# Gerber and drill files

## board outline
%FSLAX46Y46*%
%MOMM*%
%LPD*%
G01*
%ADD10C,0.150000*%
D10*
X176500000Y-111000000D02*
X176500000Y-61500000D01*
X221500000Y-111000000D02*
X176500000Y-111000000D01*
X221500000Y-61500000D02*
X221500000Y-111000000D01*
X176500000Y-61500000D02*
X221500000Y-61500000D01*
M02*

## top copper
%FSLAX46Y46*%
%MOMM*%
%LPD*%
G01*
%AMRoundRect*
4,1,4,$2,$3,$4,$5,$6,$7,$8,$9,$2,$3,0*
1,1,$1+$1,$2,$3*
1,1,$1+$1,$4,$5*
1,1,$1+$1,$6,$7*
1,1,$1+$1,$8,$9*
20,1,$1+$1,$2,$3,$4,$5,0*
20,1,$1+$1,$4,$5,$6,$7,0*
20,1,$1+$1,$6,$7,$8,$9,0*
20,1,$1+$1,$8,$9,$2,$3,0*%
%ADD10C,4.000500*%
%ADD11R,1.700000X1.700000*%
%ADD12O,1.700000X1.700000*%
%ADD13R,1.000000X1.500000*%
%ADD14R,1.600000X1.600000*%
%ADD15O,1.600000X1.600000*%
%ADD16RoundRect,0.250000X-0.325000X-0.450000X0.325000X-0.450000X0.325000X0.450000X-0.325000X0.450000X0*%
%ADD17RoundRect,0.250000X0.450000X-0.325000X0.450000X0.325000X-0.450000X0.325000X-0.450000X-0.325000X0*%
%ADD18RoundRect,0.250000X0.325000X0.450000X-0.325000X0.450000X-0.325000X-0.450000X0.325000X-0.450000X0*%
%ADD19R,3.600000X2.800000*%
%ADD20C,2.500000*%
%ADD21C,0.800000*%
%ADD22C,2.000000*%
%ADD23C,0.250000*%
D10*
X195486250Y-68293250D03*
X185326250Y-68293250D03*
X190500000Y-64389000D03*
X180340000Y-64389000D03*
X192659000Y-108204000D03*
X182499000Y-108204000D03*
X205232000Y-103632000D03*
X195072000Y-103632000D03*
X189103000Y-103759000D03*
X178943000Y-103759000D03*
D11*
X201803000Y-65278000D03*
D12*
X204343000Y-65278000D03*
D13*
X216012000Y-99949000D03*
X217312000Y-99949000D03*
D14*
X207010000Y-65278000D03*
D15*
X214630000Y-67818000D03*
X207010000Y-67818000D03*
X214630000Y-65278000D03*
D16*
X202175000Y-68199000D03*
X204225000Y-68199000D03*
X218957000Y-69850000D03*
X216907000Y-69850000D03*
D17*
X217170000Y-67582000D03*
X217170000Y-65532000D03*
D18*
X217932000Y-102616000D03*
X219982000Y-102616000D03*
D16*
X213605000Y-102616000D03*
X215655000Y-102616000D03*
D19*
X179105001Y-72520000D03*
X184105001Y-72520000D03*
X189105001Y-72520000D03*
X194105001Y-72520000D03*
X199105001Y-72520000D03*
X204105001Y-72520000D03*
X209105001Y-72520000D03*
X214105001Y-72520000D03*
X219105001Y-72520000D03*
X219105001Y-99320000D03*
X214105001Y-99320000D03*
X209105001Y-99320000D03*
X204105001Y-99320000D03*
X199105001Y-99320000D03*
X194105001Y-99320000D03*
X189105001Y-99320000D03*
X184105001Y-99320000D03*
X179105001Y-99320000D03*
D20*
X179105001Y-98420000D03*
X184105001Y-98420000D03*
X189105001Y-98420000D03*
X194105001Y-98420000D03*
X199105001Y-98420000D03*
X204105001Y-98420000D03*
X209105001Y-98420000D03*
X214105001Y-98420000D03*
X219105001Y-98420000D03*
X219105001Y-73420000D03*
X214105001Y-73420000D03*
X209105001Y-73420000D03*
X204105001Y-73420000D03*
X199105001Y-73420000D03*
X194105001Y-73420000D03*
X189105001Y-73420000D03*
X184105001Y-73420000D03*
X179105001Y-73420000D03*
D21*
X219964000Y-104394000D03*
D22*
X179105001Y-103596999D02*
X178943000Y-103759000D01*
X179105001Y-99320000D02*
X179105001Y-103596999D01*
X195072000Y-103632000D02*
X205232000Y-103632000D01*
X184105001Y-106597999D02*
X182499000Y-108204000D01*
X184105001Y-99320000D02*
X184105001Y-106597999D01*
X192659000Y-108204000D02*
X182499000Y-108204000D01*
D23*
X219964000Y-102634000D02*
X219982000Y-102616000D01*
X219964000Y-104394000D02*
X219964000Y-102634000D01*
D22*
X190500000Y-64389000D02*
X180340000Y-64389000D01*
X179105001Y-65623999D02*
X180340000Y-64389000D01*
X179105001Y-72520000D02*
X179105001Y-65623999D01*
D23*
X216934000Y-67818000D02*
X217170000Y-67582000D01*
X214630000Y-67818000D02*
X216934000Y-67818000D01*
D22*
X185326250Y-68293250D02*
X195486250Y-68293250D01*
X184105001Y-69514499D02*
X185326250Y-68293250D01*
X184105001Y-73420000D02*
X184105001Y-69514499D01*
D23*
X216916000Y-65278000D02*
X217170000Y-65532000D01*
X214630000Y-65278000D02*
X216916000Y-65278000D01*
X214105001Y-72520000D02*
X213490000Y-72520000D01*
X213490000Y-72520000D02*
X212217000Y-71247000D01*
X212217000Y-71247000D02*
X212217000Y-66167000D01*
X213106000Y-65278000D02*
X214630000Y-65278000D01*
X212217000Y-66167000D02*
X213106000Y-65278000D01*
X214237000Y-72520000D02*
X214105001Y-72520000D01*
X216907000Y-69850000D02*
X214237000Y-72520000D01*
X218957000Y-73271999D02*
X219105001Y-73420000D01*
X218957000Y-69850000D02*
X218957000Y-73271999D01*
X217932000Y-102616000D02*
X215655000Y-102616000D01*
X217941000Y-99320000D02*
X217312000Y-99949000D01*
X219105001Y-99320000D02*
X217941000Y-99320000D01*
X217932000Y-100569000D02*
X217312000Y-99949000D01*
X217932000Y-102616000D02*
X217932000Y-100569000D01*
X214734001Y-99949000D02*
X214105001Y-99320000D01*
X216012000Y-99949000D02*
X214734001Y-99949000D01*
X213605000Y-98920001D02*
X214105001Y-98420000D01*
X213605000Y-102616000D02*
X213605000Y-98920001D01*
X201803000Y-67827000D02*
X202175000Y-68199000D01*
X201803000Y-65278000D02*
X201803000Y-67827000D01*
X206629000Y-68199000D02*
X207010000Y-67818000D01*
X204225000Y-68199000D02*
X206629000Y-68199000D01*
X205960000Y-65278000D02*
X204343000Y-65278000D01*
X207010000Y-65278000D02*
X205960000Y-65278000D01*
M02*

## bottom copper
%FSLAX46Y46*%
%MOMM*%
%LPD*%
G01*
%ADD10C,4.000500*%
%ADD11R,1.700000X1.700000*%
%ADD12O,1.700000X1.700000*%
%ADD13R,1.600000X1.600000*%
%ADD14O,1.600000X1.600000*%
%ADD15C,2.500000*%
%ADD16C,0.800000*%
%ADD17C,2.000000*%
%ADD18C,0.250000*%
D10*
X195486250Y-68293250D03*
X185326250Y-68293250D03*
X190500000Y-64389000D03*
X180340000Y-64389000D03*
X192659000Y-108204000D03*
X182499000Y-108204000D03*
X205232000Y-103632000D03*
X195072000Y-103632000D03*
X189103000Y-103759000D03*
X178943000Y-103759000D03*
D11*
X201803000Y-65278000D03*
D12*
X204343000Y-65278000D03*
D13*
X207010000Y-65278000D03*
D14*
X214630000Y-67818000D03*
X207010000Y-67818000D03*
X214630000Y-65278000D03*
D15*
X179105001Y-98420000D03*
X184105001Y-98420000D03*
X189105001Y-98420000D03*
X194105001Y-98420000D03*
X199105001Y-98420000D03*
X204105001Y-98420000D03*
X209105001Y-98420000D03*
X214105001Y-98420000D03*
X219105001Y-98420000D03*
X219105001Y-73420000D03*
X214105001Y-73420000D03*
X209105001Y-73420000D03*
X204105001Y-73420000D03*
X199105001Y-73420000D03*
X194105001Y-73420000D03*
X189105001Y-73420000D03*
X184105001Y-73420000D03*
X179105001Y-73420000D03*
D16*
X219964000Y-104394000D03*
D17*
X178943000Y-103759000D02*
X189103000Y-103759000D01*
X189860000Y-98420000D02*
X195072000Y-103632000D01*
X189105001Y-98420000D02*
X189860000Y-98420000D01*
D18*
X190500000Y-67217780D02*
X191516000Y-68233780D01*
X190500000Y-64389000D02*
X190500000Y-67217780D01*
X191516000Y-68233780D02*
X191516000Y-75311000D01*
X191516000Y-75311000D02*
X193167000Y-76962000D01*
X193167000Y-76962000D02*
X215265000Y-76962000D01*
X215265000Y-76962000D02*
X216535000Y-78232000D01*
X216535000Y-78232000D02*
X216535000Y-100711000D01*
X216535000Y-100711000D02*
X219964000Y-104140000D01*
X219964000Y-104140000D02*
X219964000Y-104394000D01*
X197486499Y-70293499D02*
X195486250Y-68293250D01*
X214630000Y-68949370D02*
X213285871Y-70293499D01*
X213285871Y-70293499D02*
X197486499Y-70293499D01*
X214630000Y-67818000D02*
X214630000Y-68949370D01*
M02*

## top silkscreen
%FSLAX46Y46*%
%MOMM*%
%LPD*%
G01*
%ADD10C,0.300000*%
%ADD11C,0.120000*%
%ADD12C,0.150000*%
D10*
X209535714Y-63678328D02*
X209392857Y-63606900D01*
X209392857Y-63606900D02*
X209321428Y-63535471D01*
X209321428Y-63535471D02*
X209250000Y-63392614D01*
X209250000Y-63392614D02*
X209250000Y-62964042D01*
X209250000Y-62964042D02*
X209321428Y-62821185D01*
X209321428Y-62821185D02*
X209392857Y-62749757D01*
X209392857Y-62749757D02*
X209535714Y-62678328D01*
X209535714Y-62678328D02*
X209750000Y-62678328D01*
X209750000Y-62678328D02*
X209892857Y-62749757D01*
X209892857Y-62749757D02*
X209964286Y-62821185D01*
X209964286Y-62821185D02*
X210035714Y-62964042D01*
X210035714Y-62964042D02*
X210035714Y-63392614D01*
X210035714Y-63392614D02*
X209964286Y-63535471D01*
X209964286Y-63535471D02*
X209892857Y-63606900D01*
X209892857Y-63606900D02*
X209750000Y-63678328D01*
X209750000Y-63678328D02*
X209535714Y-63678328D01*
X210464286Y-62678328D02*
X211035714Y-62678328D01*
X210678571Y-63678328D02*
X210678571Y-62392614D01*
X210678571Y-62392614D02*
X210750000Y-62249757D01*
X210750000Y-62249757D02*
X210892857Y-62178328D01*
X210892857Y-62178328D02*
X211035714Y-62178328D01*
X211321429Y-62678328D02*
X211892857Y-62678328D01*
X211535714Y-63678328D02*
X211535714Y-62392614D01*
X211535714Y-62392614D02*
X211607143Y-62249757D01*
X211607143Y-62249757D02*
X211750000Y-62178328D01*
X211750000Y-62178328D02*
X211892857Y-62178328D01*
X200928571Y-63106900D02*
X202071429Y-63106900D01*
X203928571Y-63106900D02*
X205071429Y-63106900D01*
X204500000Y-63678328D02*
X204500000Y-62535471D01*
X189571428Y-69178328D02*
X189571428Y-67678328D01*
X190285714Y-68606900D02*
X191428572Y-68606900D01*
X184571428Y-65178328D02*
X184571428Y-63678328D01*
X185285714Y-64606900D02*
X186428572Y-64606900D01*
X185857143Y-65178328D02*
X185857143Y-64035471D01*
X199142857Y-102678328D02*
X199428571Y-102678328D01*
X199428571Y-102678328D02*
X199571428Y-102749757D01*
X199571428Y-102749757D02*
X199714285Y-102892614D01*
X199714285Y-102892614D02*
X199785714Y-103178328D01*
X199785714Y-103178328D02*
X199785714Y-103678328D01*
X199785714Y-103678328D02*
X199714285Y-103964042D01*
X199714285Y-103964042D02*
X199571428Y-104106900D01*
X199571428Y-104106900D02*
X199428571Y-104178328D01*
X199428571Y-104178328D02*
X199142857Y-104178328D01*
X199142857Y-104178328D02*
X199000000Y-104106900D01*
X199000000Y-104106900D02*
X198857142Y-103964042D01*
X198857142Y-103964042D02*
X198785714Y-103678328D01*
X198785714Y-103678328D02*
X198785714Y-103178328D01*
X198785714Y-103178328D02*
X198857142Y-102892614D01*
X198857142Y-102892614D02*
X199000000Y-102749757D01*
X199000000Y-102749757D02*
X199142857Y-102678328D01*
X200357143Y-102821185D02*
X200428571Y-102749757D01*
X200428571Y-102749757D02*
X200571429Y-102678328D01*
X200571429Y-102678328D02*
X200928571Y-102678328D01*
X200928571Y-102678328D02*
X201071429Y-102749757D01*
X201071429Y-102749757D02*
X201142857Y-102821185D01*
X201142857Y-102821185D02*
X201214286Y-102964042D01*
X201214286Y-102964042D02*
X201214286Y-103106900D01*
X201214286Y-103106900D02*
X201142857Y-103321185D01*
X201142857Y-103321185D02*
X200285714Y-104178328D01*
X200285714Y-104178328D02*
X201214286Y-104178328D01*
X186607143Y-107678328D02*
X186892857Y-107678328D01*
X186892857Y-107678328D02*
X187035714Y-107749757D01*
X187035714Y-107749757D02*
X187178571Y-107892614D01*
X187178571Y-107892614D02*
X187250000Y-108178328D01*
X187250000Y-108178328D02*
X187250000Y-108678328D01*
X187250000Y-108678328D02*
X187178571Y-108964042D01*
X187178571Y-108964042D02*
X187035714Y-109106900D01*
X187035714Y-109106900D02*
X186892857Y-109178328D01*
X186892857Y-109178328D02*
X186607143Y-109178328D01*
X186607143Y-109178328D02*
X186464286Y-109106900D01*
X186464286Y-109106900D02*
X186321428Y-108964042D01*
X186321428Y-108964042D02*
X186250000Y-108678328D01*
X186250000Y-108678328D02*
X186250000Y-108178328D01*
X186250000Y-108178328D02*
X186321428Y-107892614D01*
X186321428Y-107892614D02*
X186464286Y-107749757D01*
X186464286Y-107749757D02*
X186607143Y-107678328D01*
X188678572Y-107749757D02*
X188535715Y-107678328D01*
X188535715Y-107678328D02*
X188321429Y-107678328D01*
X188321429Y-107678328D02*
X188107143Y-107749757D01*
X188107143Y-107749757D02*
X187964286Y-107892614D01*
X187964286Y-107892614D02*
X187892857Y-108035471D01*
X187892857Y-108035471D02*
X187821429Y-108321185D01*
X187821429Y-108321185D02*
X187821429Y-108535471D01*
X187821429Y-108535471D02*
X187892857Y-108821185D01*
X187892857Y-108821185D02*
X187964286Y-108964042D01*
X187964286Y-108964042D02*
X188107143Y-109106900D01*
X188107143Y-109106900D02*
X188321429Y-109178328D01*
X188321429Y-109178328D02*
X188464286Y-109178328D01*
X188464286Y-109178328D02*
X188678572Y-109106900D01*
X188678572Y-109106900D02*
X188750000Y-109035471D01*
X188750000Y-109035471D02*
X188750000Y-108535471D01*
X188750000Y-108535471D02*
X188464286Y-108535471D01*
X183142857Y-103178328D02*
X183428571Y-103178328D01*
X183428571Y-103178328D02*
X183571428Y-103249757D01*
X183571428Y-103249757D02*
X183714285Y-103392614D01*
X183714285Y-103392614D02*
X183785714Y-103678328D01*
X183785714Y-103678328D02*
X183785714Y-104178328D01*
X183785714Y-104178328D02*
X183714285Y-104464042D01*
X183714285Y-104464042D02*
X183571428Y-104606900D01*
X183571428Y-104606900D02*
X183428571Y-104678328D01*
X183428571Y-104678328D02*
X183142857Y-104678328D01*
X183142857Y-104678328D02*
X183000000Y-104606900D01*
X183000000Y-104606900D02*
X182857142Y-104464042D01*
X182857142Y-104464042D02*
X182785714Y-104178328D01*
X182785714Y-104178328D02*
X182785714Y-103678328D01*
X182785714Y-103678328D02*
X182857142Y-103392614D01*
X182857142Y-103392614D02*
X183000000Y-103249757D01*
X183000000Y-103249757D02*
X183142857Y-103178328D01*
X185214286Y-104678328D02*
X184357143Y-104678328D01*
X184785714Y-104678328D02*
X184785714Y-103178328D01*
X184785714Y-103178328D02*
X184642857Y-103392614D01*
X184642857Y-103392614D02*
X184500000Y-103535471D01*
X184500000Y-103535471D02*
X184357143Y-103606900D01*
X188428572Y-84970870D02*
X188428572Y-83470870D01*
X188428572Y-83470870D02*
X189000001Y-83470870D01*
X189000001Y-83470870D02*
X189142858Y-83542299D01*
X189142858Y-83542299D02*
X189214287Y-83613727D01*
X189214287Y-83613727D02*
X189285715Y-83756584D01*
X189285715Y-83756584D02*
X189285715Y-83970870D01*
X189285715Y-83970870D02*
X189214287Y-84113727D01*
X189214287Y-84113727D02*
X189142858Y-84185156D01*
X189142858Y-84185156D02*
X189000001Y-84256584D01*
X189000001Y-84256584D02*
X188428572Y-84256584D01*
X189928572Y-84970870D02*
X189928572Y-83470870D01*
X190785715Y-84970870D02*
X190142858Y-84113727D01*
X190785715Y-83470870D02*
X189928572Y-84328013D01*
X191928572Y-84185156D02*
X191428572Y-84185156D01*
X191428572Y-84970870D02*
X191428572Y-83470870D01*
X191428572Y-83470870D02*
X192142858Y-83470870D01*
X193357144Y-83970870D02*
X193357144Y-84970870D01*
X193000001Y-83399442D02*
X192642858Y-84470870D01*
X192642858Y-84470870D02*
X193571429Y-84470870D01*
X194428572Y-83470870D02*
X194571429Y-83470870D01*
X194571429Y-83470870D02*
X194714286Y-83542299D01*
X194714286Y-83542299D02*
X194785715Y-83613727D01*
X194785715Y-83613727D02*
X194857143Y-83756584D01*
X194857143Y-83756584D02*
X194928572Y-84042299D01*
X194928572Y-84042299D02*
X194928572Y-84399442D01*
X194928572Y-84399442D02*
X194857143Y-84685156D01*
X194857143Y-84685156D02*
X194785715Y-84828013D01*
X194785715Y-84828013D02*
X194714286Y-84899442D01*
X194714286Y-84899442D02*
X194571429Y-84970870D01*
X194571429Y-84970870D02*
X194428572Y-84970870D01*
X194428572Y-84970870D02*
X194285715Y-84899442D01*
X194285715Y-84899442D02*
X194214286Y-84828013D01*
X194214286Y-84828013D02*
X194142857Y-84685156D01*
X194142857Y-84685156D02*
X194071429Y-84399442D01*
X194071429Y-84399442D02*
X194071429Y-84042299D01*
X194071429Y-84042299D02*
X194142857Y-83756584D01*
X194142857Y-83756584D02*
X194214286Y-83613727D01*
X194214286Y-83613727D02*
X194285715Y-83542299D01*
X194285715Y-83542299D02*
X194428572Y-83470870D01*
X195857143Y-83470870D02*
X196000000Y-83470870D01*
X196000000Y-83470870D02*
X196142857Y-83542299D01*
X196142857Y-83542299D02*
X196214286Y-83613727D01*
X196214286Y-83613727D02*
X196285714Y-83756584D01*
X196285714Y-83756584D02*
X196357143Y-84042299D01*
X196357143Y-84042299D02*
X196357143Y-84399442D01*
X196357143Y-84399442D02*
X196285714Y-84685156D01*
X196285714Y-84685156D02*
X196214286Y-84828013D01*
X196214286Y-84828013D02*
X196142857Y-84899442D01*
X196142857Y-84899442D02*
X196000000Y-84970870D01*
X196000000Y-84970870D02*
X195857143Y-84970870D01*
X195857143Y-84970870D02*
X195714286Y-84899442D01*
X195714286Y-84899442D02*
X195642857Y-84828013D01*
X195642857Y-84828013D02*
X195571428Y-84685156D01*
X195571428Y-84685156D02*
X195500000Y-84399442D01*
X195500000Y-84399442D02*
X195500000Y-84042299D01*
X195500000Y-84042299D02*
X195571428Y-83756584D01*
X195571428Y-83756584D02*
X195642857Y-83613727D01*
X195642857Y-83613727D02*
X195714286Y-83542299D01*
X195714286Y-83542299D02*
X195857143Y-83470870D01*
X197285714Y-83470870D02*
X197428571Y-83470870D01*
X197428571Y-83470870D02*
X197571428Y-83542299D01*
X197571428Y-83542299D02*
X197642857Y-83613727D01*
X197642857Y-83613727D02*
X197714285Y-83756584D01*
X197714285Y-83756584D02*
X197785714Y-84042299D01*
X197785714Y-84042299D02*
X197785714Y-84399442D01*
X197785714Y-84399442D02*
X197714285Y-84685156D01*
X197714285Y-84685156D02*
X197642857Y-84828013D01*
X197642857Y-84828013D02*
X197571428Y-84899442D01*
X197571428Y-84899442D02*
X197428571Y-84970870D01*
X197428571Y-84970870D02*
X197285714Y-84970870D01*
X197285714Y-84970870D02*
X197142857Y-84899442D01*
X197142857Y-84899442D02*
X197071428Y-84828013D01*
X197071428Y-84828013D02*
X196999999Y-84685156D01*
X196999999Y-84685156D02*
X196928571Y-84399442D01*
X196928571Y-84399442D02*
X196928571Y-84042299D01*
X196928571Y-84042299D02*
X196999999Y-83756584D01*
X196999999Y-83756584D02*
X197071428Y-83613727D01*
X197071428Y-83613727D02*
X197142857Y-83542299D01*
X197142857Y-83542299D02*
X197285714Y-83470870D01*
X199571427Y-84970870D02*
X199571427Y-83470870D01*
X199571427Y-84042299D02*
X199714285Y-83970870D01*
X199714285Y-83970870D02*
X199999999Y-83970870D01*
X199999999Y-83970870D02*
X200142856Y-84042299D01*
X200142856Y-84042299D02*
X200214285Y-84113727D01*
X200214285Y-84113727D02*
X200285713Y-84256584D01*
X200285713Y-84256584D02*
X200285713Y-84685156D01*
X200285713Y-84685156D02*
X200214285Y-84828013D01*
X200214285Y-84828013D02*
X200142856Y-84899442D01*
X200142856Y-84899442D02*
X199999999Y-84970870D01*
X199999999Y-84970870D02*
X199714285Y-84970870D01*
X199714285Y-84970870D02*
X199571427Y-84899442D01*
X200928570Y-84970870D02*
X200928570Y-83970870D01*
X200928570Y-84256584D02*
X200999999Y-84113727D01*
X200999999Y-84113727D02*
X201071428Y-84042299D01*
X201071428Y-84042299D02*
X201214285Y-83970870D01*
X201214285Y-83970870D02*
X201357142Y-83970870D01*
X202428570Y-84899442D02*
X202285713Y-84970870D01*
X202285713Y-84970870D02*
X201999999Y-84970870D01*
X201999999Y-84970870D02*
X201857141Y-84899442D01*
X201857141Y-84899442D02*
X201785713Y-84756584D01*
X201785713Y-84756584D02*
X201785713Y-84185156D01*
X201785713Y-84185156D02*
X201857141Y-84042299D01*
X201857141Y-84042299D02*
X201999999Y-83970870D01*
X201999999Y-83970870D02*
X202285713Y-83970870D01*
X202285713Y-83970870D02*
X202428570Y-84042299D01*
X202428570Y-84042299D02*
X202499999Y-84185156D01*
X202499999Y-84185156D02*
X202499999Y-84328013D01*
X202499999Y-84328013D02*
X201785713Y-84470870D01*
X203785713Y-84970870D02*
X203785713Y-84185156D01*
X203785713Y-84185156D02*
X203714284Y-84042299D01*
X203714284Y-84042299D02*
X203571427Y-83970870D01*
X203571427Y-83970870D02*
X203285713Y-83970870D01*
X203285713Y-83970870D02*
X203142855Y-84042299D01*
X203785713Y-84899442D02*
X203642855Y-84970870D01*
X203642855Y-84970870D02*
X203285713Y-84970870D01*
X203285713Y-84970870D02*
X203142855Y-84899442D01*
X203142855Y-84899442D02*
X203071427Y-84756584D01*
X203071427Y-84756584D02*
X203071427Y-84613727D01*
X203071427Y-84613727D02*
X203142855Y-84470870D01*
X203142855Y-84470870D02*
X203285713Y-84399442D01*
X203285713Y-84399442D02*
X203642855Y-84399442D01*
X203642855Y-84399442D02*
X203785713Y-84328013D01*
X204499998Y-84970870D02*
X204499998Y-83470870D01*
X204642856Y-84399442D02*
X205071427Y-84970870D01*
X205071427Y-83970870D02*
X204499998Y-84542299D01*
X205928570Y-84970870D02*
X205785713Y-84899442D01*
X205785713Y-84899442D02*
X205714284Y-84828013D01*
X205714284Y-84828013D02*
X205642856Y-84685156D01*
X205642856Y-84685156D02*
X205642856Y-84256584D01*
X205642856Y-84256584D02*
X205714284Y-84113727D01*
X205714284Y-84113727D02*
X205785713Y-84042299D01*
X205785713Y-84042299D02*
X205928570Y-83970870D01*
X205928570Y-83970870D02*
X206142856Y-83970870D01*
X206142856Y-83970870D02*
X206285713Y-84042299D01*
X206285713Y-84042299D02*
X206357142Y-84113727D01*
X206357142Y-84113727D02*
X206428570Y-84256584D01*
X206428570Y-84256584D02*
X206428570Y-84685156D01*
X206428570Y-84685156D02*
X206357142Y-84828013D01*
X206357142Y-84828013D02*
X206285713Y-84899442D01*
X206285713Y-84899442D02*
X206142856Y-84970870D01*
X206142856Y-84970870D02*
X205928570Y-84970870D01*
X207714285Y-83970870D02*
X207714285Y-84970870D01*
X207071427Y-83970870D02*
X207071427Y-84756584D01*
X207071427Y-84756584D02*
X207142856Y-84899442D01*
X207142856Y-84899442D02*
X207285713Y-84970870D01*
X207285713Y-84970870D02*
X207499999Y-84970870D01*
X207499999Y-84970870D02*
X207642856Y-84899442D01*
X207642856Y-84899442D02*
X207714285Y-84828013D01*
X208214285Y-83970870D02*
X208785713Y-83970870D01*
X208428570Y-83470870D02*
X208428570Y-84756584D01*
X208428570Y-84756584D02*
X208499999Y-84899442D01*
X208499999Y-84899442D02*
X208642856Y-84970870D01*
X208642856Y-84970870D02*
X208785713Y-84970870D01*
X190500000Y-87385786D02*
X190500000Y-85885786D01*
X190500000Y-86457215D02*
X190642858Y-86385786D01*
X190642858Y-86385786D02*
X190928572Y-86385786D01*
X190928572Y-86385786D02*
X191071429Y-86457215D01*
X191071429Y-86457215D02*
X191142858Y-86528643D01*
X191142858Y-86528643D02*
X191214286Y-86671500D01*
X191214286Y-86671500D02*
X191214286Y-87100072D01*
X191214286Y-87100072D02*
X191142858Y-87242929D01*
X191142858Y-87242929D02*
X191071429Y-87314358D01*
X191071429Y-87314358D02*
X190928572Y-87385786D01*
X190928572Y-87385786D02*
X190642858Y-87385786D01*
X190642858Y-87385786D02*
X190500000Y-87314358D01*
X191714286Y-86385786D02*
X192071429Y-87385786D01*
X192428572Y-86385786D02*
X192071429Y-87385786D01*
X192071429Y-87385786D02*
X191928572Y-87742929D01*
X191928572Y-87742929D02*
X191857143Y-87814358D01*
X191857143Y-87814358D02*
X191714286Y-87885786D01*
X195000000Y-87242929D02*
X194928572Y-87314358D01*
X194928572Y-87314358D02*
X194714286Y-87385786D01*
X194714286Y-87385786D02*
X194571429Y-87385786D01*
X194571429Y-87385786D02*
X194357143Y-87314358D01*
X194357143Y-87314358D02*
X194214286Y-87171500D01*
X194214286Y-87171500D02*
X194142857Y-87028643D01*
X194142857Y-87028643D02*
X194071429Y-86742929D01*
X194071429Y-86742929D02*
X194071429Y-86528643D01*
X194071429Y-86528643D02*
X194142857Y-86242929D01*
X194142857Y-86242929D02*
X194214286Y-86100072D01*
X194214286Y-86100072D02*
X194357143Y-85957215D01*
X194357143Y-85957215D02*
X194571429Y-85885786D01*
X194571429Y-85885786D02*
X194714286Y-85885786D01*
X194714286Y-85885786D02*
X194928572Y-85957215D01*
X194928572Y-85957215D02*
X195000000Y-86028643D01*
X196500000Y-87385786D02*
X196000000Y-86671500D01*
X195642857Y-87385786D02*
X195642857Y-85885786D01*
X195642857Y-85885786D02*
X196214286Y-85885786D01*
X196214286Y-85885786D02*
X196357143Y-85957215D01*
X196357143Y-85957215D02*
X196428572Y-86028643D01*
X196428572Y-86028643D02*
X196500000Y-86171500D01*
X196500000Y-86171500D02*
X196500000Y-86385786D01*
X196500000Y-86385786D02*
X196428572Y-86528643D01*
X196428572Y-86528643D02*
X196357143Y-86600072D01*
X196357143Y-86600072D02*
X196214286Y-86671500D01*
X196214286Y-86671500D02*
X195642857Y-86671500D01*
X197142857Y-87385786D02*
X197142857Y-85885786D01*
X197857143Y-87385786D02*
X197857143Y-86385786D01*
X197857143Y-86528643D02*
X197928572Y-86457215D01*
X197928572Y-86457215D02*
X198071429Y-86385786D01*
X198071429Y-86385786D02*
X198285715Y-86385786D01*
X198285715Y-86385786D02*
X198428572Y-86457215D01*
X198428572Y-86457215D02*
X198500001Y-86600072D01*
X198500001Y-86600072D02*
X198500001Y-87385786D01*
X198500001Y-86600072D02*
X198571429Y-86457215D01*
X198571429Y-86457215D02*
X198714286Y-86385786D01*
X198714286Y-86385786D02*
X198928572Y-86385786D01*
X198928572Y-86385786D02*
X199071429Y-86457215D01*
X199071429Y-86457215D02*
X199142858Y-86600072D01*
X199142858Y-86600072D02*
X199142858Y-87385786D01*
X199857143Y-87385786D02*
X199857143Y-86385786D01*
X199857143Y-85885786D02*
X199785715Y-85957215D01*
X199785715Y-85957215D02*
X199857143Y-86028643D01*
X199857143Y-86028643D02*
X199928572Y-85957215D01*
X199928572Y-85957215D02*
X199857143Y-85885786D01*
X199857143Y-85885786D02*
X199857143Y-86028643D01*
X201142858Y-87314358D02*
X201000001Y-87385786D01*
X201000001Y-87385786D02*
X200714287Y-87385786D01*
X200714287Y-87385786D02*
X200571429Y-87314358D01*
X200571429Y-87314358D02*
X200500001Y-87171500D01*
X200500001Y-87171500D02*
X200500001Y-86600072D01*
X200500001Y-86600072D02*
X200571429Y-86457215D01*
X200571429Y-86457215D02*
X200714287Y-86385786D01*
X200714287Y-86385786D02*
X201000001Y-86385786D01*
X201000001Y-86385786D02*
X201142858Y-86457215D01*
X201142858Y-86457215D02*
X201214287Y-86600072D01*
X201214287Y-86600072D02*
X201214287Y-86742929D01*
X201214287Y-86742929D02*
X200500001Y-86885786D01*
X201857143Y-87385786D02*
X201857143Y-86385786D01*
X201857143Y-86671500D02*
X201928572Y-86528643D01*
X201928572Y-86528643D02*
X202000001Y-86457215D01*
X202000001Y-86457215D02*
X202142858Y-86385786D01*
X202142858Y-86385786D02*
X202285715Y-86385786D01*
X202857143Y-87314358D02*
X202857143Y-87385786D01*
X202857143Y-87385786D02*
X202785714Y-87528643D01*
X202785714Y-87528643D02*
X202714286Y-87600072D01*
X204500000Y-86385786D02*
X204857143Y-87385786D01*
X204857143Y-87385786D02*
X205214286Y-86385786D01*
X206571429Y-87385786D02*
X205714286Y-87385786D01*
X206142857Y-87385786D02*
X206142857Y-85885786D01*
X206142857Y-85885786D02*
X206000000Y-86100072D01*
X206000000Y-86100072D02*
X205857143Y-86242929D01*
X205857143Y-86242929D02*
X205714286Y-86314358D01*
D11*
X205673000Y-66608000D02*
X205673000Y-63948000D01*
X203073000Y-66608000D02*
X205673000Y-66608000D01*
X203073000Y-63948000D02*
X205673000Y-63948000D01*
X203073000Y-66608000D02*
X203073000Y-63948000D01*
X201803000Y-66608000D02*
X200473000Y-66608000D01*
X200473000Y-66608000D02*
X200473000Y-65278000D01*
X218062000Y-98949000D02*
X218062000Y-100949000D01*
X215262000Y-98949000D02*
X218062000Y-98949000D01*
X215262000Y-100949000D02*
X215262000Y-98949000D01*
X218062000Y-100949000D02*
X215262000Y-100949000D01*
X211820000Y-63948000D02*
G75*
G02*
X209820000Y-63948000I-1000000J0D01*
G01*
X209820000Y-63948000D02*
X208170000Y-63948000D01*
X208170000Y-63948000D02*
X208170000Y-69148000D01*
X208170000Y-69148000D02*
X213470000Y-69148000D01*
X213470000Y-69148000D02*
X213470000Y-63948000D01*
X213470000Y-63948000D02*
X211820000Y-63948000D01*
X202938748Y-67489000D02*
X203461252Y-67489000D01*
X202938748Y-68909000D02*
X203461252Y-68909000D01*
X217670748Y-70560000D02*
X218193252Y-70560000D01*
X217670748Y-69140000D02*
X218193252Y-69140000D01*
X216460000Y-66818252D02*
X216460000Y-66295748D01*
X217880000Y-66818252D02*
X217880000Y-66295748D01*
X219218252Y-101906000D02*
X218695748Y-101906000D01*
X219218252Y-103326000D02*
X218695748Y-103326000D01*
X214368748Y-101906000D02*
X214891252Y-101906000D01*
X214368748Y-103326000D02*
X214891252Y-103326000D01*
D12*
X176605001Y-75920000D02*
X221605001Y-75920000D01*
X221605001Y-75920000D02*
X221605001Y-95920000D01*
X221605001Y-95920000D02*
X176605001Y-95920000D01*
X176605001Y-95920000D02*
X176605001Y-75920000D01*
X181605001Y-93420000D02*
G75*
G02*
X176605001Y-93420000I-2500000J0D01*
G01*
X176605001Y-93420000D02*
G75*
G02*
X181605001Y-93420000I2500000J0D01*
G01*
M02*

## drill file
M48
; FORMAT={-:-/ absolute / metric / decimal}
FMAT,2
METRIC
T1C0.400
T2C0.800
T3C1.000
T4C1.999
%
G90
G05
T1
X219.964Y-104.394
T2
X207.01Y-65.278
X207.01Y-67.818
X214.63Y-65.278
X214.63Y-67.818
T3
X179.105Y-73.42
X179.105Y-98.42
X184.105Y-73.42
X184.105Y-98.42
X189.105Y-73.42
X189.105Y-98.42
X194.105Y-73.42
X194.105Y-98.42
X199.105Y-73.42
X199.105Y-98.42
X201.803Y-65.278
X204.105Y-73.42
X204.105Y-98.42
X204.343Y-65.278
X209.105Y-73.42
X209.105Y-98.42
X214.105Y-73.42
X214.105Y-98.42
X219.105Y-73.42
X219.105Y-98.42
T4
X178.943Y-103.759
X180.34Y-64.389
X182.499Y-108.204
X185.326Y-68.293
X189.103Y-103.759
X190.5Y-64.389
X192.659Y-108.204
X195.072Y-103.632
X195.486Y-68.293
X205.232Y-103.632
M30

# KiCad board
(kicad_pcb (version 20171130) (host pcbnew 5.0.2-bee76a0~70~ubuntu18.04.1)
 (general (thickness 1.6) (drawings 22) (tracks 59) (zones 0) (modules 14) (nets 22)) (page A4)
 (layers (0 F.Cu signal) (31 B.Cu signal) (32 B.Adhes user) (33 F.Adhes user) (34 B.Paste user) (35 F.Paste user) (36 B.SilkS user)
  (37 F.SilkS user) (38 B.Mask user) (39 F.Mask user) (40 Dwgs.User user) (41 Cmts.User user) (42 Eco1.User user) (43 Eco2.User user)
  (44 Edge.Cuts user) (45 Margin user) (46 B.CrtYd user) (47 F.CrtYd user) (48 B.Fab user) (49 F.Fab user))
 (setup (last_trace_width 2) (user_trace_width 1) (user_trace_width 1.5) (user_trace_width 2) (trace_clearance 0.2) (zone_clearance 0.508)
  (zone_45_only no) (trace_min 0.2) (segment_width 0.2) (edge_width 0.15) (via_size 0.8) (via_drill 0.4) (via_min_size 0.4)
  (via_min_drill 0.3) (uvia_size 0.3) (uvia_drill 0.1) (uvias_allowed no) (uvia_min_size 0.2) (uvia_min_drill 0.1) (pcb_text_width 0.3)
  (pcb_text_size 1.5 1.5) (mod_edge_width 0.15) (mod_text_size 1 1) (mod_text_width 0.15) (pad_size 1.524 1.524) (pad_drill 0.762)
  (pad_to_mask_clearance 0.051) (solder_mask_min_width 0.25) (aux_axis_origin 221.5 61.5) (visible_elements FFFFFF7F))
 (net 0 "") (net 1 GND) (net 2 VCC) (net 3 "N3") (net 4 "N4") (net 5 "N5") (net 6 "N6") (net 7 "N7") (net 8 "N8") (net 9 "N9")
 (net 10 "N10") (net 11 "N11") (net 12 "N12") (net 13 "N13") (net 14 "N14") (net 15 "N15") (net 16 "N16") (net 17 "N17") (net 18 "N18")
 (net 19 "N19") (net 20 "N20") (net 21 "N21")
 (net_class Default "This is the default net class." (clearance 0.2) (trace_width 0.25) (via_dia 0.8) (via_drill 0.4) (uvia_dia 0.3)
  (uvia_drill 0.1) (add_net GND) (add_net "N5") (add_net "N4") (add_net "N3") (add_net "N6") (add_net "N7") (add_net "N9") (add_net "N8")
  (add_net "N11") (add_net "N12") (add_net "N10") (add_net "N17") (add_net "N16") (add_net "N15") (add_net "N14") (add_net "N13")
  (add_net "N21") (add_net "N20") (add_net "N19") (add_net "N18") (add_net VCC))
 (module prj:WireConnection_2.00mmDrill (layer F.Cu) (at 185.32625 68.29325)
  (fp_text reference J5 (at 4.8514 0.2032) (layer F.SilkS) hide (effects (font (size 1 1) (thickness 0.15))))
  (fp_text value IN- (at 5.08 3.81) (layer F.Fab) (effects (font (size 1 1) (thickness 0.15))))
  (pad 1 thru_hole circle (at 10.16 0) (size 4.0005 4.0005) (drill 1.99898) (layers *.Cu *.Mask) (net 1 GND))
  (pad 1 thru_hole circle (at 0 0) (size 4.0005 4.0005) (drill 1.99898) (layers *.Cu *.Mask) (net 1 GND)))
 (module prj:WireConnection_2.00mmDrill (layer F.Cu) (at 180.34 64.389)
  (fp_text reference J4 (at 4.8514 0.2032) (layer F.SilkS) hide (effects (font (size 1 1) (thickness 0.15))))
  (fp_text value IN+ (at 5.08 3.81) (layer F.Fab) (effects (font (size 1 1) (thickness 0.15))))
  (pad 1 thru_hole circle (at 10.16 0) (size 4.0005 4.0005) (drill 1.99898) (layers *.Cu *.Mask) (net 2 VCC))
  (pad 1 thru_hole circle (at 0 0) (size 4.0005 4.0005) (drill 1.99898) (layers *.Cu *.Mask) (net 2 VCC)))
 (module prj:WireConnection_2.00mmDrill (layer F.Cu) (at 182.499 108.204)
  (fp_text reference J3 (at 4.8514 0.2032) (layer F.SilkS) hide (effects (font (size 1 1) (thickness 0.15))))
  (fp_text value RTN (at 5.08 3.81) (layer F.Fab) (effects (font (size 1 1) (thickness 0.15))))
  (pad 1 thru_hole circle (at 10.16 0) (size 4.0005 4.0005) (drill 1.99898) (layers *.Cu *.Mask) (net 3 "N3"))
  (pad 1 thru_hole circle (at 0 0) (size 4.0005 4.0005) (drill 1.99898) (layers *.Cu *.Mask) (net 3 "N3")))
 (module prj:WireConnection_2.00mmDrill (layer F.Cu) (at 195.072 103.632)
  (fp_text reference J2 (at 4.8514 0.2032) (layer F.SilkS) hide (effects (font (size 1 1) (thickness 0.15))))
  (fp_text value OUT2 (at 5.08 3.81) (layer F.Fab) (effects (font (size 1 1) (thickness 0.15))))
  (pad 1 thru_hole circle (at 10.16 0) (size 4.0005 4.0005) (drill 1.99898) (layers *.Cu *.Mask) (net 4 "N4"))
  (pad 1 thru_hole circle (at 0 0) (size 4.0005 4.0005) (drill 1.99898) (layers *.Cu *.Mask) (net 4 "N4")))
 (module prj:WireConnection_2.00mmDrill (layer F.Cu) (at 178.943 103.759)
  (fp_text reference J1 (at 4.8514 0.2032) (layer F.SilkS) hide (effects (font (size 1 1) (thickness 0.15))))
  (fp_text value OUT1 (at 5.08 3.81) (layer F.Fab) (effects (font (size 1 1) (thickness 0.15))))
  (pad 1 thru_hole circle (at 10.16 0) (size 4.0005 4.0005) (drill 1.99898) (layers *.Cu *.Mask) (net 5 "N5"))
  (pad 1 thru_hole circle (at 0 0) (size 4.0005 4.0005) (drill 1.99898) (layers *.Cu *.Mask) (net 5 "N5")))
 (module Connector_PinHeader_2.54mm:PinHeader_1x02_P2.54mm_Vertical (layer F.Cu) (at 201.803 65.278 90)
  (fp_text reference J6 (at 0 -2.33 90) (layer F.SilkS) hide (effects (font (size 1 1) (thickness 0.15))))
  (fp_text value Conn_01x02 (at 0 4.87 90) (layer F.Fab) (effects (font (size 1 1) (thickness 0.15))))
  (fp_line (start -1.33 3.87) (end 1.33 3.87) (layer F.SilkS) (width 0.12))
  (fp_line (start -1.33 1.27) (end -1.33 3.87) (layer F.SilkS) (width 0.12))
  (fp_line (start 1.33 1.27) (end 1.33 3.87) (layer F.SilkS) (width 0.12))
  (fp_line (start -1.33 1.27) (end 1.33 1.27) (layer F.SilkS) (width 0.12))
  (fp_line (start -1.33 0) (end -1.33 -1.33) (layer F.SilkS) (width 0.12))
  (fp_line (start -1.33 -1.33) (end 0 -1.33) (layer F.SilkS) (width 0.12))
  (pad 1 thru_hole rect (at 0 0 90) (size 1.7 1.7) (drill 1) (layers *.Cu *.Mask) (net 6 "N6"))
  (pad 2 thru_hole oval (at 0 2.54 90) (size 1.7 1.7) (drill 1) (layers *.Cu *.Mask) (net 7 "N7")))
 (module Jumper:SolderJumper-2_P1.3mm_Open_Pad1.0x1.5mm (layer F.Cu) (at 216.662 99.949 180)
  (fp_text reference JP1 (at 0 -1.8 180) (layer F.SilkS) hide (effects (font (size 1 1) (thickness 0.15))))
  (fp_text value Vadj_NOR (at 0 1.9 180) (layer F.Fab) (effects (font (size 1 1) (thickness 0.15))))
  (fp_line (start -1.4 1) (end -1.4 -1) (layer F.SilkS) (width 0.12))
  (fp_line (start 1.4 1) (end -1.4 1) (layer F.SilkS) (width 0.12))
  (fp_line (start 1.4 -1) (end 1.4 1) (layer F.SilkS) (width 0.12))
  (fp_line (start -1.4 -1) (end 1.4 -1) (layer F.SilkS) (width 0.12))
  (pad 2 smd rect (at 0.65 0 180) (size 1 1.5) (layers F.Cu F.Mask) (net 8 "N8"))
  (pad 1 smd rect (at -0.65 0 180) (size 1 1.5) (layers F.Cu F.Mask) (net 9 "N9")))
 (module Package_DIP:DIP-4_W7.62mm (layer F.Cu) (at 207.01 65.278)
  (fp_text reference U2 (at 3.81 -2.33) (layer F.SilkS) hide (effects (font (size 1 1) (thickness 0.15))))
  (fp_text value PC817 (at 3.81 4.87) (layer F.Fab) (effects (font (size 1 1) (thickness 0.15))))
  (fp_arc (start 3.81 -1.33) (end 2.81 -1.33) (angle -180) (layer F.SilkS) (width 0.12))
  (fp_line (start 2.81 -1.33) (end 1.16 -1.33) (layer F.SilkS) (width 0.12))
  (fp_line (start 1.16 -1.33) (end 1.16 3.87) (layer F.SilkS) (width 0.12))
  (fp_line (start 1.16 3.87) (end 6.46 3.87) (layer F.SilkS) (width 0.12))
  (fp_line (start 6.46 3.87) (end 6.46 -1.33) (layer F.SilkS) (width 0.12))
  (fp_line (start 6.46 -1.33) (end 4.81 -1.33) (layer F.SilkS) (width 0.12))
  (pad 1 thru_hole rect (at 0 0) (size 1.6 1.6) (drill 0.8) (layers *.Cu *.Mask) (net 7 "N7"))
  (pad 3 thru_hole oval (at 7.62 2.54) (size 1.6 1.6) (drill 0.8) (layers *.Cu *.Mask) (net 1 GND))
  (pad 2 thru_hole oval (at 0 2.54) (size 1.6 1.6) (drill 0.8) (layers *.Cu *.Mask) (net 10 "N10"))
  (pad 4 thru_hole oval (at 7.62 0) (size 1.6 1.6) (drill 0.8) (layers *.Cu *.Mask) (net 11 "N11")))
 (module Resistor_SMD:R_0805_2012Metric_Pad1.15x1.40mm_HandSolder (layer F.Cu) (at 203.2 68.199)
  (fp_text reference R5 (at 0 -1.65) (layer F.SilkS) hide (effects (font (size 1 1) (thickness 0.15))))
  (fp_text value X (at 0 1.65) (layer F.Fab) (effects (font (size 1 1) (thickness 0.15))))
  (fp_line (start -0.261252 -0.71) (end 0.261252 -0.71) (layer F.SilkS) (width 0.12))
  (fp_line (start -0.261252 0.71) (end 0.261252 0.71) (layer F.SilkS) (width 0.12))
  (pad 1 smd roundrect (at -1.025 0) (size 1.15 1.4) (layers F.Cu F.Paste F.Mask) (roundrect_rratio 0.217391) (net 6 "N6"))
  (pad 2 smd roundrect (at 1.025 0) (size 1.15 1.4) (layers F.Cu F.Paste F.Mask) (roundrect_rratio 0.217391) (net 10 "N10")))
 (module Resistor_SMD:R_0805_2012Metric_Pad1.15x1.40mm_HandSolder (layer F.Cu) (at 217.932 69.85)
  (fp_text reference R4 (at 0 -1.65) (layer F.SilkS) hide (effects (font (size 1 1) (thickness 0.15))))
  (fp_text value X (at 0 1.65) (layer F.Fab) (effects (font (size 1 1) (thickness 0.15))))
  (fp_line (start -0.261252 0.71) (end 0.261252 0.71) (layer F.SilkS) (width 0.12))
  (fp_line (start -0.261252 -0.71) (end 0.261252 -0.71) (layer F.SilkS) (width 0.12))
  (pad 2 smd roundrect (at 1.025 0) (size 1.15 1.4) (layers F.Cu F.Paste F.Mask) (roundrect_rratio 0.217391) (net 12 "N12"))
  (pad 1 smd roundrect (at -1.025 0) (size 1.15 1.4) (layers F.Cu F.Paste F.Mask) (roundrect_rratio 0.217391) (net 11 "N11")))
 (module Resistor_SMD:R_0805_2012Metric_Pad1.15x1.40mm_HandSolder (layer F.Cu) (at 217.17 66.557 90)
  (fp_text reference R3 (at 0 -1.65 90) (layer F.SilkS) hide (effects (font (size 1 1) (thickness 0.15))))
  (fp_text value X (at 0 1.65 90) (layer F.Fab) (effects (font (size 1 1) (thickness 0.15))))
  (fp_line (start -0.261252 -0.71) (end 0.261252 -0.71) (layer F.SilkS) (width 0.12))
  (fp_line (start -0.261252 0.71) (end 0.261252 0.71) (layer F.SilkS) (width 0.12))
  (pad 1 smd roundrect (at -1.025 0 90) (size 1.15 1.4) (layers F.Cu F.Paste F.Mask) (roundrect_rratio 0.217391) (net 1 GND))
  (pad 2 smd roundrect (at 1.025 0 90) (size 1.15 1.4) (layers F.Cu F.Paste F.Mask) (roundrect_rratio 0.217391) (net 11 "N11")))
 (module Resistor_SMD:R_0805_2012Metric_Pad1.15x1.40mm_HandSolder (layer F.Cu) (at 218.957 102.616 180)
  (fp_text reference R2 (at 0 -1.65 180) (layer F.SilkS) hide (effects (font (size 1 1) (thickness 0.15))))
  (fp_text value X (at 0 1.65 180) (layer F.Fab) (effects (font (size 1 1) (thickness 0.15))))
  (fp_line (start -0.261252 0.71) (end 0.261252 0.71) (layer F.SilkS) (width 0.12))
  (fp_line (start -0.261252 -0.71) (end 0.261252 -0.71) (layer F.SilkS) (width 0.12))
  (pad 2 smd roundrect (at 1.025 0 180) (size 1.15 1.4) (layers F.Cu F.Paste F.Mask) (roundrect_rratio 0.217391) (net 9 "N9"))
  (pad 1 smd roundrect (at -1.025 0 180) (size 1.15 1.4) (layers F.Cu F.Paste F.Mask) (roundrect_rratio 0.217391) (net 2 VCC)))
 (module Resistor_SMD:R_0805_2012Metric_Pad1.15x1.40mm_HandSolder (layer F.Cu) (at 214.63 102.616)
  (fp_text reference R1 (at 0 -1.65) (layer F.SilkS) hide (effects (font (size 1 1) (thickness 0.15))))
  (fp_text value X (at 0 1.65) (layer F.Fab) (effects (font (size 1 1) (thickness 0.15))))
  (fp_line (start -0.261252 -0.71) (end 0.261252 -0.71) (layer F.SilkS) (width 0.12))
  (fp_line (start -0.261252 0.71) (end 0.261252 0.71) (layer F.SilkS) (width 0.12))
  (pad 1 smd roundrect (at -1.025 0) (size 1.15 1.4) (layers F.Cu F.Paste F.Mask) (roundrect_rratio 0.217391) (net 8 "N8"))
  (pad 2 smd roundrect (at 1.025 0) (size 1.15 1.4) (layers F.Cu F.Paste F.Mask) (roundrect_rratio 0.217391) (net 9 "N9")))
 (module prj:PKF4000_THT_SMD (layer F.Cu) (at 199.105001 85.92)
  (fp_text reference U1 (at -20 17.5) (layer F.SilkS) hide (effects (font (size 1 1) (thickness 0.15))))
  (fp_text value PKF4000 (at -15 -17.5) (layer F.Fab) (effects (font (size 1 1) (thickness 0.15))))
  (fp_line (start -22.5 -10) (end 22.5 -10) (layer F.SilkS) (width 0.15))
  (fp_line (start 22.5 -10) (end 22.5 10) (layer F.SilkS) (width 0.15))
  (fp_line (start 22.5 10) (end -22.5 10) (layer F.SilkS) (width 0.15))
  (fp_line (start -22.5 10) (end -22.5 -10) (layer F.SilkS) (width 0.15))
  (fp_circle (center -20 7.5) (end -20 10) (layer F.SilkS) (width 0.15))
  (pad 18 smd rect (at -20 -13.4) (size 3.6 2.8) (layers F.Cu F.Paste F.Mask) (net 2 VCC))
  (pad 17 smd rect (at -15 -13.4) (size 3.6 2.8) (layers F.Cu F.Paste F.Mask) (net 1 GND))
  (pad 16 smd rect (at -10 -13.4) (size 3.6 2.8) (layers F.Cu F.Paste F.Mask) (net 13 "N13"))
  (pad 15 smd rect (at -5 -13.4) (size 3.6 2.8) (layers F.Cu F.Paste F.Mask) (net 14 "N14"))
  (pad 14 smd rect (at 0 -13.4) (size 3.6 2.8) (layers F.Cu F.Paste F.Mask) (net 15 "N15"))
  (pad 13 smd rect (at 5 -13.4) (size 3.6 2.8) (layers F.Cu F.Paste F.Mask) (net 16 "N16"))
  (pad 12 smd rect (at 10 -13.4) (size 3.6 2.8) (layers F.Cu F.Paste F.Mask) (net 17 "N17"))
  (pad 11 smd rect (at 15 -13.4) (size 3.6 2.8) (layers F.Cu F.Paste F.Mask) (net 11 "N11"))
  (pad 10 smd rect (at 20 -13.4) (size 3.6 2.8) (layers F.Cu F.Paste F.Mask) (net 12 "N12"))
  (pad 9 smd rect (at 20 13.4) (size 3.6 2.8) (layers F.Cu F.Paste F.Mask) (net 9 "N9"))
  (pad 8 smd rect (at 15 13.4) (size 3.6 2.8) (layers F.Cu F.Paste F.Mask) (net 8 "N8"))
  (pad 7 smd rect (at 10 13.4) (size 3.6 2.8) (layers F.Cu F.Paste F.Mask) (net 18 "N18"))
  (pad 6 smd rect (at 5 13.4) (size 3.6 2.8) (layers F.Cu F.Paste F.Mask) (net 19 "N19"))
  (pad 5 smd rect (at 0 13.4) (size 3.6 2.8) (layers F.Cu F.Paste F.Mask) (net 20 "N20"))
  (pad 4 smd rect (at -5 13.4) (size 3.6 2.8) (layers F.Cu F.Paste F.Mask) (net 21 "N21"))
  (pad 3 smd rect (at -10 13.4) (size 3.6 2.8) (layers F.Cu F.Paste F.Mask) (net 4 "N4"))
  (pad 2 smd rect (at -15 13.4) (size 3.6 2.8) (layers F.Cu F.Paste F.Mask) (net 3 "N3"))
  (pad 1 smd rect (at -20 13.4) (size 3.6 2.8) (layers F.Cu F.Paste F.Mask) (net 5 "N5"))
  (pad 1 thru_hole circle (at -20 12.5) (size 2.5 2.5) (drill 1) (layers *.Cu *.Mask) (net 5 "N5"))
  (pad 2 thru_hole circle (at -15 12.5) (size 2.5 2.5) (drill 1) (layers *.Cu *.Mask) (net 3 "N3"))
  (pad 3 thru_hole circle (at -10 12.5) (size 2.5 2.5) (drill 1) (layers *.Cu *.Mask) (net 4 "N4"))
  (pad 4 thru_hole circle (at -5 12.5) (size 2.5 2.5) (drill 1) (layers *.Cu *.Mask) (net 21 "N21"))
  (pad 5 thru_hole circle (at 0 12.5) (size 2.5 2.5) (drill 1) (layers *.Cu *.Mask) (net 20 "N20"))
  (pad 6 thru_hole circle (at 5 12.5) (size 2.5 2.5) (drill 1) (layers *.Cu *.Mask) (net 19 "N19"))
  (pad 7 thru_hole circle (at 10 12.5) (size 2.5 2.5) (drill 1) (layers *.Cu *.Mask) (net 18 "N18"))
  (pad 8 thru_hole circle (at 15 12.5) (size 2.5 2.5) (drill 1) (layers *.Cu *.Mask) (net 8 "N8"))
  (pad 9 thru_hole circle (at 20 12.5) (size 2.5 2.5) (drill 1) (layers *.Cu *.Mask) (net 9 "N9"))
  (pad 10 thru_hole circle (at 20 -12.5) (size 2.5 2.5) (drill 1) (layers *.Cu *.Mask) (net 12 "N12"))
  (pad 11 thru_hole circle (at 15 -12.5) (size 2.5 2.5) (drill 1) (layers *.Cu *.Mask) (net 11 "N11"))
  (pad 12 thru_hole circle (at 10 -12.5) (size 2.5 2.5) (drill 1) (layers *.Cu *.Mask) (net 17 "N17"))
  (pad 13 thru_hole circle (at 5 -12.5) (size 2.5 2.5) (drill 1) (layers *.Cu *.Mask) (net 16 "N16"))
  (pad 14 thru_hole circle (at 0 -12.5) (size 2.5 2.5) (drill 1) (layers *.Cu *.Mask) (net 15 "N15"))
  (pad 15 thru_hole circle (at -5 -12.5) (size 2.5 2.5) (drill 1) (layers *.Cu *.Mask) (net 14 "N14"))
  (pad 16 thru_hole circle (at -10 -12.5) (size 2.5 2.5) (drill 1) (layers *.Cu *.Mask) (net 13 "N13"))
  (pad 17 thru_hole circle (at -15 -12.5) (size 2.5 2.5) (drill 1) (layers *.Cu *.Mask) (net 1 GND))
  (pad 18 thru_hole circle (at -20 -12.5) (size 2.5 2.5) (drill 1) (layers *.Cu *.Mask) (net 2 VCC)))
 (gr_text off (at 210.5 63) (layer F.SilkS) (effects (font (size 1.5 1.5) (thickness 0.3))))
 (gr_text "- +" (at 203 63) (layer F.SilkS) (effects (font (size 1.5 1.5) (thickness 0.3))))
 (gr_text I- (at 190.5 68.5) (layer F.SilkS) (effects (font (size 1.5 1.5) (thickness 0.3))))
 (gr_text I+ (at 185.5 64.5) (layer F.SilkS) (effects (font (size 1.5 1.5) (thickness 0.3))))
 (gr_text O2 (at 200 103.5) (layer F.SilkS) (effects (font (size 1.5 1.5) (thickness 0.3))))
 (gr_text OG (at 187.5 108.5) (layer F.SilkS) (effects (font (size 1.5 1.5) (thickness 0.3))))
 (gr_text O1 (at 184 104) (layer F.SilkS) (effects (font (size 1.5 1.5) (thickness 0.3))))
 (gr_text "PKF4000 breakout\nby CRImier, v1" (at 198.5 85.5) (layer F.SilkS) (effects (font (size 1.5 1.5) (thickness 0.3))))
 (gr_line (start 176.5 111) (end 176.5 61.5) (layer Edge.Cuts) (width 0.15))
 (gr_line (start 221.5 111) (end 176.5 111) (layer Edge.Cuts) (width 0.15))
 (gr_line (start 221.5 61.5) (end 221.5 111) (layer Edge.Cuts) (width 0.15))
 (gr_line (start 176.5 61.5) (end 221.5 61.5) (layer Edge.Cuts) (width 0.15))
 (segment (start 178.943 103.759) (end 189.103 103.759) (width 2) (layer B.Cu) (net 5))
 (segment (start 179.105001 103.596999) (end 178.943 103.759) (width 2) (layer F.Cu) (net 5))
 (segment (start 179.105001 99.32) (end 179.105001 103.596999) (width 2) (layer F.Cu) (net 5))
 (segment (start 195.072 103.632) (end 205.232 103.632) (width 2) (layer F.Cu) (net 4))
 (segment (start 189.86 98.42) (end 195.072 103.632) (width 2) (layer B.Cu) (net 4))
 (segment (start 189.105001 98.42) (end 189.86 98.42) (width 2) (layer B.Cu) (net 4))
 (segment (start 184.105001 106.597999) (end 182.499 108.204) (width 2) (layer F.Cu) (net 3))
 (segment (start 184.105001 99.32) (end 184.105001 106.597999) (width 2) (layer F.Cu) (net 3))
 (segment (start 192.659 108.204) (end 182.499 108.204) (width 2) (layer F.Cu) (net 3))
 (segment (start 190.5 67.21778) (end 191.516 68.23378) (width 0.25) (layer B.Cu) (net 2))
 (segment (start 190.5 64.389) (end 190.5 67.21778) (width 0.25) (layer B.Cu) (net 2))
 (segment (start 191.516 68.23378) (end 191.516 75.311) (width 0.25) (layer B.Cu) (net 2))
 (segment (start 191.516 75.311) (end 193.167 76.962) (width 0.25) (layer B.Cu) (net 2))
 (segment (start 193.167 76.962) (end 215.265 76.962) (width 0.25) (layer B.Cu) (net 2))
 (segment (start 215.265 76.962) (end 216.535 78.232) (width 0.25) (layer B.Cu) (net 2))
 (segment (start 216.535 78.232) (end 216.535 100.711) (width 0.25) (layer B.Cu) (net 2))
 (via (at 219.964 104.394) (size 0.8) (drill 0.4) (layers F.Cu B.Cu) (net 2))
 (segment (start 216.535 100.711) (end 219.964 104.14) (width 0.25) (layer B.Cu) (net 2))
 (segment (start 219.964 104.14) (end 219.964 104.394) (width 0.25) (layer B.Cu) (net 2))
 (segment (start 219.964 102.634) (end 219.982 102.616) (width 0.25) (layer F.Cu) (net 2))
 (segment (start 219.964 104.394) (end 219.964 102.634) (width 0.25) (layer F.Cu) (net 2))
 (segment (start 190.5 64.389) (end 180.34 64.389) (width 2) (layer F.Cu) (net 2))
 (segment (start 179.105001 65.623999) (end 180.34 64.389) (width 2) (layer F.Cu) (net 2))
 (segment (start 179.105001 72.52) (end 179.105001 65.623999) (width 2) (layer F.Cu) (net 2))
 (segment (start 216.934 67.818) (end 217.17 67.582) (width 0.25) (layer F.Cu) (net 1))
 (segment (start 214.63 67.818) (end 216.934 67.818) (width 0.25) (layer F.Cu) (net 1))
 (segment (start 197.486499 70.293499) (end 195.48625 68.29325) (width 0.25) (layer B.Cu) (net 1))
 (segment (start 214.63 68.94937) (end 213.285871 70.293499) (width 0.25) (layer B.Cu) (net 1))
 (segment (start 213.285871 70.293499) (end 197.486499 70.293499) (width 0.25) (layer B.Cu) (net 1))
 (segment (start 214.63 67.818) (end 214.63 68.94937) (width 0.25) (layer B.Cu) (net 1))
 (segment (start 185.32625 68.29325) (end 195.48625 68.29325) (width 2) (layer F.Cu) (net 1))
 (segment (start 184.105001 69.514499) (end 185.32625 68.29325) (width 2) (layer F.Cu) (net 1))
 (segment (start 184.105001 73.42) (end 184.105001 69.514499) (width 2) (layer F.Cu) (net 1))
 (segment (start 216.916 65.278) (end 217.17 65.532) (width 0.25) (layer F.Cu) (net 11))
 (segment (start 214.63 65.278) (end 216.916 65.278) (width 0.25) (layer F.Cu) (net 11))
 (segment (start 214.105001 72.52) (end 213.49 72.52) (width 0.25) (layer F.Cu) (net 11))
 (segment (start 213.49 72.52) (end 212.217 71.247) (width 0.25) (layer F.Cu) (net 11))
 (segment (start 212.217 71.247) (end 212.217 66.167) (width 0.25) (layer F.Cu) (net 11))
 (segment (start 213.106 65.278) (end 214.63 65.278) (width 0.25) (layer F.Cu) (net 11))
 (segment (start 212.217 66.167) (end 213.106 65.278) (width 0.25) (layer F.Cu) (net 11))
 (segment (start 214.237 72.52) (end 214.105001 72.52) (width 0.25) (layer F.Cu) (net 11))
 (segment (start 216.907 69.85) (end 214.237 72.52) (width 0.25) (layer F.Cu) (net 11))
 (segment (start 218.957 73.271999) (end 219.105001 73.42) (width 0.25) (layer F.Cu) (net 12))
 (segment (start 218.957 69.85) (end 218.957 73.271999) (width 0.25) (layer F.Cu) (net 12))
 (segment (start 217.932 102.616) (end 215.655 102.616) (width 0.25) (layer F.Cu) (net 9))
 (segment (start 217.941 99.32) (end 217.312 99.949) (width 0.25) (layer F.Cu) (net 9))
 (segment (start 219.105001 99.32) (end 217.941 99.32) (width 0.25) (layer F.Cu) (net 9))
 (segment (start 217.932 100.569) (end 217.312 99.949) (width 0.25) (layer F.Cu) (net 9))
 (segment (start 217.932 102.616) (end 217.932 100.569) (width 0.25) (layer F.Cu) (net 9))
 (segment (start 214.734001 99.949) (end 214.105001 99.32) (width 0.25) (layer F.Cu) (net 8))
 (segment (start 216.012 99.949) (end 214.734001 99.949) (width 0.25) (layer F.Cu) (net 8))
 (segment (start 213.605 98.920001) (end 214.105001 98.42) (width 0.25) (layer F.Cu) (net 8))
 (segment (start 213.605 102.616) (end 213.605 98.920001) (width 0.25) (layer F.Cu) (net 8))
 (segment (start 201.803 67.827) (end 202.175 68.199) (width 0.25) (layer F.Cu) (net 6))
 (segment (start 201.803 65.278) (end 201.803 67.827) (width 0.25) (layer F.Cu) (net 6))
 (segment (start 206.629 68.199) (end 207.01 67.818) (width 0.25) (layer F.Cu) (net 10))
 (segment (start 204.225 68.199) (end 206.629 68.199) (width 0.25) (layer F.Cu) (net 10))
 (segment (start 205.96 65.278) (end 204.343 65.278) (width 0.25) (layer F.Cu) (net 7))
 (segment (start 207.01 65.278) (end 205.96 65.278) (width 0.25) (layer F.Cu) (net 7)))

